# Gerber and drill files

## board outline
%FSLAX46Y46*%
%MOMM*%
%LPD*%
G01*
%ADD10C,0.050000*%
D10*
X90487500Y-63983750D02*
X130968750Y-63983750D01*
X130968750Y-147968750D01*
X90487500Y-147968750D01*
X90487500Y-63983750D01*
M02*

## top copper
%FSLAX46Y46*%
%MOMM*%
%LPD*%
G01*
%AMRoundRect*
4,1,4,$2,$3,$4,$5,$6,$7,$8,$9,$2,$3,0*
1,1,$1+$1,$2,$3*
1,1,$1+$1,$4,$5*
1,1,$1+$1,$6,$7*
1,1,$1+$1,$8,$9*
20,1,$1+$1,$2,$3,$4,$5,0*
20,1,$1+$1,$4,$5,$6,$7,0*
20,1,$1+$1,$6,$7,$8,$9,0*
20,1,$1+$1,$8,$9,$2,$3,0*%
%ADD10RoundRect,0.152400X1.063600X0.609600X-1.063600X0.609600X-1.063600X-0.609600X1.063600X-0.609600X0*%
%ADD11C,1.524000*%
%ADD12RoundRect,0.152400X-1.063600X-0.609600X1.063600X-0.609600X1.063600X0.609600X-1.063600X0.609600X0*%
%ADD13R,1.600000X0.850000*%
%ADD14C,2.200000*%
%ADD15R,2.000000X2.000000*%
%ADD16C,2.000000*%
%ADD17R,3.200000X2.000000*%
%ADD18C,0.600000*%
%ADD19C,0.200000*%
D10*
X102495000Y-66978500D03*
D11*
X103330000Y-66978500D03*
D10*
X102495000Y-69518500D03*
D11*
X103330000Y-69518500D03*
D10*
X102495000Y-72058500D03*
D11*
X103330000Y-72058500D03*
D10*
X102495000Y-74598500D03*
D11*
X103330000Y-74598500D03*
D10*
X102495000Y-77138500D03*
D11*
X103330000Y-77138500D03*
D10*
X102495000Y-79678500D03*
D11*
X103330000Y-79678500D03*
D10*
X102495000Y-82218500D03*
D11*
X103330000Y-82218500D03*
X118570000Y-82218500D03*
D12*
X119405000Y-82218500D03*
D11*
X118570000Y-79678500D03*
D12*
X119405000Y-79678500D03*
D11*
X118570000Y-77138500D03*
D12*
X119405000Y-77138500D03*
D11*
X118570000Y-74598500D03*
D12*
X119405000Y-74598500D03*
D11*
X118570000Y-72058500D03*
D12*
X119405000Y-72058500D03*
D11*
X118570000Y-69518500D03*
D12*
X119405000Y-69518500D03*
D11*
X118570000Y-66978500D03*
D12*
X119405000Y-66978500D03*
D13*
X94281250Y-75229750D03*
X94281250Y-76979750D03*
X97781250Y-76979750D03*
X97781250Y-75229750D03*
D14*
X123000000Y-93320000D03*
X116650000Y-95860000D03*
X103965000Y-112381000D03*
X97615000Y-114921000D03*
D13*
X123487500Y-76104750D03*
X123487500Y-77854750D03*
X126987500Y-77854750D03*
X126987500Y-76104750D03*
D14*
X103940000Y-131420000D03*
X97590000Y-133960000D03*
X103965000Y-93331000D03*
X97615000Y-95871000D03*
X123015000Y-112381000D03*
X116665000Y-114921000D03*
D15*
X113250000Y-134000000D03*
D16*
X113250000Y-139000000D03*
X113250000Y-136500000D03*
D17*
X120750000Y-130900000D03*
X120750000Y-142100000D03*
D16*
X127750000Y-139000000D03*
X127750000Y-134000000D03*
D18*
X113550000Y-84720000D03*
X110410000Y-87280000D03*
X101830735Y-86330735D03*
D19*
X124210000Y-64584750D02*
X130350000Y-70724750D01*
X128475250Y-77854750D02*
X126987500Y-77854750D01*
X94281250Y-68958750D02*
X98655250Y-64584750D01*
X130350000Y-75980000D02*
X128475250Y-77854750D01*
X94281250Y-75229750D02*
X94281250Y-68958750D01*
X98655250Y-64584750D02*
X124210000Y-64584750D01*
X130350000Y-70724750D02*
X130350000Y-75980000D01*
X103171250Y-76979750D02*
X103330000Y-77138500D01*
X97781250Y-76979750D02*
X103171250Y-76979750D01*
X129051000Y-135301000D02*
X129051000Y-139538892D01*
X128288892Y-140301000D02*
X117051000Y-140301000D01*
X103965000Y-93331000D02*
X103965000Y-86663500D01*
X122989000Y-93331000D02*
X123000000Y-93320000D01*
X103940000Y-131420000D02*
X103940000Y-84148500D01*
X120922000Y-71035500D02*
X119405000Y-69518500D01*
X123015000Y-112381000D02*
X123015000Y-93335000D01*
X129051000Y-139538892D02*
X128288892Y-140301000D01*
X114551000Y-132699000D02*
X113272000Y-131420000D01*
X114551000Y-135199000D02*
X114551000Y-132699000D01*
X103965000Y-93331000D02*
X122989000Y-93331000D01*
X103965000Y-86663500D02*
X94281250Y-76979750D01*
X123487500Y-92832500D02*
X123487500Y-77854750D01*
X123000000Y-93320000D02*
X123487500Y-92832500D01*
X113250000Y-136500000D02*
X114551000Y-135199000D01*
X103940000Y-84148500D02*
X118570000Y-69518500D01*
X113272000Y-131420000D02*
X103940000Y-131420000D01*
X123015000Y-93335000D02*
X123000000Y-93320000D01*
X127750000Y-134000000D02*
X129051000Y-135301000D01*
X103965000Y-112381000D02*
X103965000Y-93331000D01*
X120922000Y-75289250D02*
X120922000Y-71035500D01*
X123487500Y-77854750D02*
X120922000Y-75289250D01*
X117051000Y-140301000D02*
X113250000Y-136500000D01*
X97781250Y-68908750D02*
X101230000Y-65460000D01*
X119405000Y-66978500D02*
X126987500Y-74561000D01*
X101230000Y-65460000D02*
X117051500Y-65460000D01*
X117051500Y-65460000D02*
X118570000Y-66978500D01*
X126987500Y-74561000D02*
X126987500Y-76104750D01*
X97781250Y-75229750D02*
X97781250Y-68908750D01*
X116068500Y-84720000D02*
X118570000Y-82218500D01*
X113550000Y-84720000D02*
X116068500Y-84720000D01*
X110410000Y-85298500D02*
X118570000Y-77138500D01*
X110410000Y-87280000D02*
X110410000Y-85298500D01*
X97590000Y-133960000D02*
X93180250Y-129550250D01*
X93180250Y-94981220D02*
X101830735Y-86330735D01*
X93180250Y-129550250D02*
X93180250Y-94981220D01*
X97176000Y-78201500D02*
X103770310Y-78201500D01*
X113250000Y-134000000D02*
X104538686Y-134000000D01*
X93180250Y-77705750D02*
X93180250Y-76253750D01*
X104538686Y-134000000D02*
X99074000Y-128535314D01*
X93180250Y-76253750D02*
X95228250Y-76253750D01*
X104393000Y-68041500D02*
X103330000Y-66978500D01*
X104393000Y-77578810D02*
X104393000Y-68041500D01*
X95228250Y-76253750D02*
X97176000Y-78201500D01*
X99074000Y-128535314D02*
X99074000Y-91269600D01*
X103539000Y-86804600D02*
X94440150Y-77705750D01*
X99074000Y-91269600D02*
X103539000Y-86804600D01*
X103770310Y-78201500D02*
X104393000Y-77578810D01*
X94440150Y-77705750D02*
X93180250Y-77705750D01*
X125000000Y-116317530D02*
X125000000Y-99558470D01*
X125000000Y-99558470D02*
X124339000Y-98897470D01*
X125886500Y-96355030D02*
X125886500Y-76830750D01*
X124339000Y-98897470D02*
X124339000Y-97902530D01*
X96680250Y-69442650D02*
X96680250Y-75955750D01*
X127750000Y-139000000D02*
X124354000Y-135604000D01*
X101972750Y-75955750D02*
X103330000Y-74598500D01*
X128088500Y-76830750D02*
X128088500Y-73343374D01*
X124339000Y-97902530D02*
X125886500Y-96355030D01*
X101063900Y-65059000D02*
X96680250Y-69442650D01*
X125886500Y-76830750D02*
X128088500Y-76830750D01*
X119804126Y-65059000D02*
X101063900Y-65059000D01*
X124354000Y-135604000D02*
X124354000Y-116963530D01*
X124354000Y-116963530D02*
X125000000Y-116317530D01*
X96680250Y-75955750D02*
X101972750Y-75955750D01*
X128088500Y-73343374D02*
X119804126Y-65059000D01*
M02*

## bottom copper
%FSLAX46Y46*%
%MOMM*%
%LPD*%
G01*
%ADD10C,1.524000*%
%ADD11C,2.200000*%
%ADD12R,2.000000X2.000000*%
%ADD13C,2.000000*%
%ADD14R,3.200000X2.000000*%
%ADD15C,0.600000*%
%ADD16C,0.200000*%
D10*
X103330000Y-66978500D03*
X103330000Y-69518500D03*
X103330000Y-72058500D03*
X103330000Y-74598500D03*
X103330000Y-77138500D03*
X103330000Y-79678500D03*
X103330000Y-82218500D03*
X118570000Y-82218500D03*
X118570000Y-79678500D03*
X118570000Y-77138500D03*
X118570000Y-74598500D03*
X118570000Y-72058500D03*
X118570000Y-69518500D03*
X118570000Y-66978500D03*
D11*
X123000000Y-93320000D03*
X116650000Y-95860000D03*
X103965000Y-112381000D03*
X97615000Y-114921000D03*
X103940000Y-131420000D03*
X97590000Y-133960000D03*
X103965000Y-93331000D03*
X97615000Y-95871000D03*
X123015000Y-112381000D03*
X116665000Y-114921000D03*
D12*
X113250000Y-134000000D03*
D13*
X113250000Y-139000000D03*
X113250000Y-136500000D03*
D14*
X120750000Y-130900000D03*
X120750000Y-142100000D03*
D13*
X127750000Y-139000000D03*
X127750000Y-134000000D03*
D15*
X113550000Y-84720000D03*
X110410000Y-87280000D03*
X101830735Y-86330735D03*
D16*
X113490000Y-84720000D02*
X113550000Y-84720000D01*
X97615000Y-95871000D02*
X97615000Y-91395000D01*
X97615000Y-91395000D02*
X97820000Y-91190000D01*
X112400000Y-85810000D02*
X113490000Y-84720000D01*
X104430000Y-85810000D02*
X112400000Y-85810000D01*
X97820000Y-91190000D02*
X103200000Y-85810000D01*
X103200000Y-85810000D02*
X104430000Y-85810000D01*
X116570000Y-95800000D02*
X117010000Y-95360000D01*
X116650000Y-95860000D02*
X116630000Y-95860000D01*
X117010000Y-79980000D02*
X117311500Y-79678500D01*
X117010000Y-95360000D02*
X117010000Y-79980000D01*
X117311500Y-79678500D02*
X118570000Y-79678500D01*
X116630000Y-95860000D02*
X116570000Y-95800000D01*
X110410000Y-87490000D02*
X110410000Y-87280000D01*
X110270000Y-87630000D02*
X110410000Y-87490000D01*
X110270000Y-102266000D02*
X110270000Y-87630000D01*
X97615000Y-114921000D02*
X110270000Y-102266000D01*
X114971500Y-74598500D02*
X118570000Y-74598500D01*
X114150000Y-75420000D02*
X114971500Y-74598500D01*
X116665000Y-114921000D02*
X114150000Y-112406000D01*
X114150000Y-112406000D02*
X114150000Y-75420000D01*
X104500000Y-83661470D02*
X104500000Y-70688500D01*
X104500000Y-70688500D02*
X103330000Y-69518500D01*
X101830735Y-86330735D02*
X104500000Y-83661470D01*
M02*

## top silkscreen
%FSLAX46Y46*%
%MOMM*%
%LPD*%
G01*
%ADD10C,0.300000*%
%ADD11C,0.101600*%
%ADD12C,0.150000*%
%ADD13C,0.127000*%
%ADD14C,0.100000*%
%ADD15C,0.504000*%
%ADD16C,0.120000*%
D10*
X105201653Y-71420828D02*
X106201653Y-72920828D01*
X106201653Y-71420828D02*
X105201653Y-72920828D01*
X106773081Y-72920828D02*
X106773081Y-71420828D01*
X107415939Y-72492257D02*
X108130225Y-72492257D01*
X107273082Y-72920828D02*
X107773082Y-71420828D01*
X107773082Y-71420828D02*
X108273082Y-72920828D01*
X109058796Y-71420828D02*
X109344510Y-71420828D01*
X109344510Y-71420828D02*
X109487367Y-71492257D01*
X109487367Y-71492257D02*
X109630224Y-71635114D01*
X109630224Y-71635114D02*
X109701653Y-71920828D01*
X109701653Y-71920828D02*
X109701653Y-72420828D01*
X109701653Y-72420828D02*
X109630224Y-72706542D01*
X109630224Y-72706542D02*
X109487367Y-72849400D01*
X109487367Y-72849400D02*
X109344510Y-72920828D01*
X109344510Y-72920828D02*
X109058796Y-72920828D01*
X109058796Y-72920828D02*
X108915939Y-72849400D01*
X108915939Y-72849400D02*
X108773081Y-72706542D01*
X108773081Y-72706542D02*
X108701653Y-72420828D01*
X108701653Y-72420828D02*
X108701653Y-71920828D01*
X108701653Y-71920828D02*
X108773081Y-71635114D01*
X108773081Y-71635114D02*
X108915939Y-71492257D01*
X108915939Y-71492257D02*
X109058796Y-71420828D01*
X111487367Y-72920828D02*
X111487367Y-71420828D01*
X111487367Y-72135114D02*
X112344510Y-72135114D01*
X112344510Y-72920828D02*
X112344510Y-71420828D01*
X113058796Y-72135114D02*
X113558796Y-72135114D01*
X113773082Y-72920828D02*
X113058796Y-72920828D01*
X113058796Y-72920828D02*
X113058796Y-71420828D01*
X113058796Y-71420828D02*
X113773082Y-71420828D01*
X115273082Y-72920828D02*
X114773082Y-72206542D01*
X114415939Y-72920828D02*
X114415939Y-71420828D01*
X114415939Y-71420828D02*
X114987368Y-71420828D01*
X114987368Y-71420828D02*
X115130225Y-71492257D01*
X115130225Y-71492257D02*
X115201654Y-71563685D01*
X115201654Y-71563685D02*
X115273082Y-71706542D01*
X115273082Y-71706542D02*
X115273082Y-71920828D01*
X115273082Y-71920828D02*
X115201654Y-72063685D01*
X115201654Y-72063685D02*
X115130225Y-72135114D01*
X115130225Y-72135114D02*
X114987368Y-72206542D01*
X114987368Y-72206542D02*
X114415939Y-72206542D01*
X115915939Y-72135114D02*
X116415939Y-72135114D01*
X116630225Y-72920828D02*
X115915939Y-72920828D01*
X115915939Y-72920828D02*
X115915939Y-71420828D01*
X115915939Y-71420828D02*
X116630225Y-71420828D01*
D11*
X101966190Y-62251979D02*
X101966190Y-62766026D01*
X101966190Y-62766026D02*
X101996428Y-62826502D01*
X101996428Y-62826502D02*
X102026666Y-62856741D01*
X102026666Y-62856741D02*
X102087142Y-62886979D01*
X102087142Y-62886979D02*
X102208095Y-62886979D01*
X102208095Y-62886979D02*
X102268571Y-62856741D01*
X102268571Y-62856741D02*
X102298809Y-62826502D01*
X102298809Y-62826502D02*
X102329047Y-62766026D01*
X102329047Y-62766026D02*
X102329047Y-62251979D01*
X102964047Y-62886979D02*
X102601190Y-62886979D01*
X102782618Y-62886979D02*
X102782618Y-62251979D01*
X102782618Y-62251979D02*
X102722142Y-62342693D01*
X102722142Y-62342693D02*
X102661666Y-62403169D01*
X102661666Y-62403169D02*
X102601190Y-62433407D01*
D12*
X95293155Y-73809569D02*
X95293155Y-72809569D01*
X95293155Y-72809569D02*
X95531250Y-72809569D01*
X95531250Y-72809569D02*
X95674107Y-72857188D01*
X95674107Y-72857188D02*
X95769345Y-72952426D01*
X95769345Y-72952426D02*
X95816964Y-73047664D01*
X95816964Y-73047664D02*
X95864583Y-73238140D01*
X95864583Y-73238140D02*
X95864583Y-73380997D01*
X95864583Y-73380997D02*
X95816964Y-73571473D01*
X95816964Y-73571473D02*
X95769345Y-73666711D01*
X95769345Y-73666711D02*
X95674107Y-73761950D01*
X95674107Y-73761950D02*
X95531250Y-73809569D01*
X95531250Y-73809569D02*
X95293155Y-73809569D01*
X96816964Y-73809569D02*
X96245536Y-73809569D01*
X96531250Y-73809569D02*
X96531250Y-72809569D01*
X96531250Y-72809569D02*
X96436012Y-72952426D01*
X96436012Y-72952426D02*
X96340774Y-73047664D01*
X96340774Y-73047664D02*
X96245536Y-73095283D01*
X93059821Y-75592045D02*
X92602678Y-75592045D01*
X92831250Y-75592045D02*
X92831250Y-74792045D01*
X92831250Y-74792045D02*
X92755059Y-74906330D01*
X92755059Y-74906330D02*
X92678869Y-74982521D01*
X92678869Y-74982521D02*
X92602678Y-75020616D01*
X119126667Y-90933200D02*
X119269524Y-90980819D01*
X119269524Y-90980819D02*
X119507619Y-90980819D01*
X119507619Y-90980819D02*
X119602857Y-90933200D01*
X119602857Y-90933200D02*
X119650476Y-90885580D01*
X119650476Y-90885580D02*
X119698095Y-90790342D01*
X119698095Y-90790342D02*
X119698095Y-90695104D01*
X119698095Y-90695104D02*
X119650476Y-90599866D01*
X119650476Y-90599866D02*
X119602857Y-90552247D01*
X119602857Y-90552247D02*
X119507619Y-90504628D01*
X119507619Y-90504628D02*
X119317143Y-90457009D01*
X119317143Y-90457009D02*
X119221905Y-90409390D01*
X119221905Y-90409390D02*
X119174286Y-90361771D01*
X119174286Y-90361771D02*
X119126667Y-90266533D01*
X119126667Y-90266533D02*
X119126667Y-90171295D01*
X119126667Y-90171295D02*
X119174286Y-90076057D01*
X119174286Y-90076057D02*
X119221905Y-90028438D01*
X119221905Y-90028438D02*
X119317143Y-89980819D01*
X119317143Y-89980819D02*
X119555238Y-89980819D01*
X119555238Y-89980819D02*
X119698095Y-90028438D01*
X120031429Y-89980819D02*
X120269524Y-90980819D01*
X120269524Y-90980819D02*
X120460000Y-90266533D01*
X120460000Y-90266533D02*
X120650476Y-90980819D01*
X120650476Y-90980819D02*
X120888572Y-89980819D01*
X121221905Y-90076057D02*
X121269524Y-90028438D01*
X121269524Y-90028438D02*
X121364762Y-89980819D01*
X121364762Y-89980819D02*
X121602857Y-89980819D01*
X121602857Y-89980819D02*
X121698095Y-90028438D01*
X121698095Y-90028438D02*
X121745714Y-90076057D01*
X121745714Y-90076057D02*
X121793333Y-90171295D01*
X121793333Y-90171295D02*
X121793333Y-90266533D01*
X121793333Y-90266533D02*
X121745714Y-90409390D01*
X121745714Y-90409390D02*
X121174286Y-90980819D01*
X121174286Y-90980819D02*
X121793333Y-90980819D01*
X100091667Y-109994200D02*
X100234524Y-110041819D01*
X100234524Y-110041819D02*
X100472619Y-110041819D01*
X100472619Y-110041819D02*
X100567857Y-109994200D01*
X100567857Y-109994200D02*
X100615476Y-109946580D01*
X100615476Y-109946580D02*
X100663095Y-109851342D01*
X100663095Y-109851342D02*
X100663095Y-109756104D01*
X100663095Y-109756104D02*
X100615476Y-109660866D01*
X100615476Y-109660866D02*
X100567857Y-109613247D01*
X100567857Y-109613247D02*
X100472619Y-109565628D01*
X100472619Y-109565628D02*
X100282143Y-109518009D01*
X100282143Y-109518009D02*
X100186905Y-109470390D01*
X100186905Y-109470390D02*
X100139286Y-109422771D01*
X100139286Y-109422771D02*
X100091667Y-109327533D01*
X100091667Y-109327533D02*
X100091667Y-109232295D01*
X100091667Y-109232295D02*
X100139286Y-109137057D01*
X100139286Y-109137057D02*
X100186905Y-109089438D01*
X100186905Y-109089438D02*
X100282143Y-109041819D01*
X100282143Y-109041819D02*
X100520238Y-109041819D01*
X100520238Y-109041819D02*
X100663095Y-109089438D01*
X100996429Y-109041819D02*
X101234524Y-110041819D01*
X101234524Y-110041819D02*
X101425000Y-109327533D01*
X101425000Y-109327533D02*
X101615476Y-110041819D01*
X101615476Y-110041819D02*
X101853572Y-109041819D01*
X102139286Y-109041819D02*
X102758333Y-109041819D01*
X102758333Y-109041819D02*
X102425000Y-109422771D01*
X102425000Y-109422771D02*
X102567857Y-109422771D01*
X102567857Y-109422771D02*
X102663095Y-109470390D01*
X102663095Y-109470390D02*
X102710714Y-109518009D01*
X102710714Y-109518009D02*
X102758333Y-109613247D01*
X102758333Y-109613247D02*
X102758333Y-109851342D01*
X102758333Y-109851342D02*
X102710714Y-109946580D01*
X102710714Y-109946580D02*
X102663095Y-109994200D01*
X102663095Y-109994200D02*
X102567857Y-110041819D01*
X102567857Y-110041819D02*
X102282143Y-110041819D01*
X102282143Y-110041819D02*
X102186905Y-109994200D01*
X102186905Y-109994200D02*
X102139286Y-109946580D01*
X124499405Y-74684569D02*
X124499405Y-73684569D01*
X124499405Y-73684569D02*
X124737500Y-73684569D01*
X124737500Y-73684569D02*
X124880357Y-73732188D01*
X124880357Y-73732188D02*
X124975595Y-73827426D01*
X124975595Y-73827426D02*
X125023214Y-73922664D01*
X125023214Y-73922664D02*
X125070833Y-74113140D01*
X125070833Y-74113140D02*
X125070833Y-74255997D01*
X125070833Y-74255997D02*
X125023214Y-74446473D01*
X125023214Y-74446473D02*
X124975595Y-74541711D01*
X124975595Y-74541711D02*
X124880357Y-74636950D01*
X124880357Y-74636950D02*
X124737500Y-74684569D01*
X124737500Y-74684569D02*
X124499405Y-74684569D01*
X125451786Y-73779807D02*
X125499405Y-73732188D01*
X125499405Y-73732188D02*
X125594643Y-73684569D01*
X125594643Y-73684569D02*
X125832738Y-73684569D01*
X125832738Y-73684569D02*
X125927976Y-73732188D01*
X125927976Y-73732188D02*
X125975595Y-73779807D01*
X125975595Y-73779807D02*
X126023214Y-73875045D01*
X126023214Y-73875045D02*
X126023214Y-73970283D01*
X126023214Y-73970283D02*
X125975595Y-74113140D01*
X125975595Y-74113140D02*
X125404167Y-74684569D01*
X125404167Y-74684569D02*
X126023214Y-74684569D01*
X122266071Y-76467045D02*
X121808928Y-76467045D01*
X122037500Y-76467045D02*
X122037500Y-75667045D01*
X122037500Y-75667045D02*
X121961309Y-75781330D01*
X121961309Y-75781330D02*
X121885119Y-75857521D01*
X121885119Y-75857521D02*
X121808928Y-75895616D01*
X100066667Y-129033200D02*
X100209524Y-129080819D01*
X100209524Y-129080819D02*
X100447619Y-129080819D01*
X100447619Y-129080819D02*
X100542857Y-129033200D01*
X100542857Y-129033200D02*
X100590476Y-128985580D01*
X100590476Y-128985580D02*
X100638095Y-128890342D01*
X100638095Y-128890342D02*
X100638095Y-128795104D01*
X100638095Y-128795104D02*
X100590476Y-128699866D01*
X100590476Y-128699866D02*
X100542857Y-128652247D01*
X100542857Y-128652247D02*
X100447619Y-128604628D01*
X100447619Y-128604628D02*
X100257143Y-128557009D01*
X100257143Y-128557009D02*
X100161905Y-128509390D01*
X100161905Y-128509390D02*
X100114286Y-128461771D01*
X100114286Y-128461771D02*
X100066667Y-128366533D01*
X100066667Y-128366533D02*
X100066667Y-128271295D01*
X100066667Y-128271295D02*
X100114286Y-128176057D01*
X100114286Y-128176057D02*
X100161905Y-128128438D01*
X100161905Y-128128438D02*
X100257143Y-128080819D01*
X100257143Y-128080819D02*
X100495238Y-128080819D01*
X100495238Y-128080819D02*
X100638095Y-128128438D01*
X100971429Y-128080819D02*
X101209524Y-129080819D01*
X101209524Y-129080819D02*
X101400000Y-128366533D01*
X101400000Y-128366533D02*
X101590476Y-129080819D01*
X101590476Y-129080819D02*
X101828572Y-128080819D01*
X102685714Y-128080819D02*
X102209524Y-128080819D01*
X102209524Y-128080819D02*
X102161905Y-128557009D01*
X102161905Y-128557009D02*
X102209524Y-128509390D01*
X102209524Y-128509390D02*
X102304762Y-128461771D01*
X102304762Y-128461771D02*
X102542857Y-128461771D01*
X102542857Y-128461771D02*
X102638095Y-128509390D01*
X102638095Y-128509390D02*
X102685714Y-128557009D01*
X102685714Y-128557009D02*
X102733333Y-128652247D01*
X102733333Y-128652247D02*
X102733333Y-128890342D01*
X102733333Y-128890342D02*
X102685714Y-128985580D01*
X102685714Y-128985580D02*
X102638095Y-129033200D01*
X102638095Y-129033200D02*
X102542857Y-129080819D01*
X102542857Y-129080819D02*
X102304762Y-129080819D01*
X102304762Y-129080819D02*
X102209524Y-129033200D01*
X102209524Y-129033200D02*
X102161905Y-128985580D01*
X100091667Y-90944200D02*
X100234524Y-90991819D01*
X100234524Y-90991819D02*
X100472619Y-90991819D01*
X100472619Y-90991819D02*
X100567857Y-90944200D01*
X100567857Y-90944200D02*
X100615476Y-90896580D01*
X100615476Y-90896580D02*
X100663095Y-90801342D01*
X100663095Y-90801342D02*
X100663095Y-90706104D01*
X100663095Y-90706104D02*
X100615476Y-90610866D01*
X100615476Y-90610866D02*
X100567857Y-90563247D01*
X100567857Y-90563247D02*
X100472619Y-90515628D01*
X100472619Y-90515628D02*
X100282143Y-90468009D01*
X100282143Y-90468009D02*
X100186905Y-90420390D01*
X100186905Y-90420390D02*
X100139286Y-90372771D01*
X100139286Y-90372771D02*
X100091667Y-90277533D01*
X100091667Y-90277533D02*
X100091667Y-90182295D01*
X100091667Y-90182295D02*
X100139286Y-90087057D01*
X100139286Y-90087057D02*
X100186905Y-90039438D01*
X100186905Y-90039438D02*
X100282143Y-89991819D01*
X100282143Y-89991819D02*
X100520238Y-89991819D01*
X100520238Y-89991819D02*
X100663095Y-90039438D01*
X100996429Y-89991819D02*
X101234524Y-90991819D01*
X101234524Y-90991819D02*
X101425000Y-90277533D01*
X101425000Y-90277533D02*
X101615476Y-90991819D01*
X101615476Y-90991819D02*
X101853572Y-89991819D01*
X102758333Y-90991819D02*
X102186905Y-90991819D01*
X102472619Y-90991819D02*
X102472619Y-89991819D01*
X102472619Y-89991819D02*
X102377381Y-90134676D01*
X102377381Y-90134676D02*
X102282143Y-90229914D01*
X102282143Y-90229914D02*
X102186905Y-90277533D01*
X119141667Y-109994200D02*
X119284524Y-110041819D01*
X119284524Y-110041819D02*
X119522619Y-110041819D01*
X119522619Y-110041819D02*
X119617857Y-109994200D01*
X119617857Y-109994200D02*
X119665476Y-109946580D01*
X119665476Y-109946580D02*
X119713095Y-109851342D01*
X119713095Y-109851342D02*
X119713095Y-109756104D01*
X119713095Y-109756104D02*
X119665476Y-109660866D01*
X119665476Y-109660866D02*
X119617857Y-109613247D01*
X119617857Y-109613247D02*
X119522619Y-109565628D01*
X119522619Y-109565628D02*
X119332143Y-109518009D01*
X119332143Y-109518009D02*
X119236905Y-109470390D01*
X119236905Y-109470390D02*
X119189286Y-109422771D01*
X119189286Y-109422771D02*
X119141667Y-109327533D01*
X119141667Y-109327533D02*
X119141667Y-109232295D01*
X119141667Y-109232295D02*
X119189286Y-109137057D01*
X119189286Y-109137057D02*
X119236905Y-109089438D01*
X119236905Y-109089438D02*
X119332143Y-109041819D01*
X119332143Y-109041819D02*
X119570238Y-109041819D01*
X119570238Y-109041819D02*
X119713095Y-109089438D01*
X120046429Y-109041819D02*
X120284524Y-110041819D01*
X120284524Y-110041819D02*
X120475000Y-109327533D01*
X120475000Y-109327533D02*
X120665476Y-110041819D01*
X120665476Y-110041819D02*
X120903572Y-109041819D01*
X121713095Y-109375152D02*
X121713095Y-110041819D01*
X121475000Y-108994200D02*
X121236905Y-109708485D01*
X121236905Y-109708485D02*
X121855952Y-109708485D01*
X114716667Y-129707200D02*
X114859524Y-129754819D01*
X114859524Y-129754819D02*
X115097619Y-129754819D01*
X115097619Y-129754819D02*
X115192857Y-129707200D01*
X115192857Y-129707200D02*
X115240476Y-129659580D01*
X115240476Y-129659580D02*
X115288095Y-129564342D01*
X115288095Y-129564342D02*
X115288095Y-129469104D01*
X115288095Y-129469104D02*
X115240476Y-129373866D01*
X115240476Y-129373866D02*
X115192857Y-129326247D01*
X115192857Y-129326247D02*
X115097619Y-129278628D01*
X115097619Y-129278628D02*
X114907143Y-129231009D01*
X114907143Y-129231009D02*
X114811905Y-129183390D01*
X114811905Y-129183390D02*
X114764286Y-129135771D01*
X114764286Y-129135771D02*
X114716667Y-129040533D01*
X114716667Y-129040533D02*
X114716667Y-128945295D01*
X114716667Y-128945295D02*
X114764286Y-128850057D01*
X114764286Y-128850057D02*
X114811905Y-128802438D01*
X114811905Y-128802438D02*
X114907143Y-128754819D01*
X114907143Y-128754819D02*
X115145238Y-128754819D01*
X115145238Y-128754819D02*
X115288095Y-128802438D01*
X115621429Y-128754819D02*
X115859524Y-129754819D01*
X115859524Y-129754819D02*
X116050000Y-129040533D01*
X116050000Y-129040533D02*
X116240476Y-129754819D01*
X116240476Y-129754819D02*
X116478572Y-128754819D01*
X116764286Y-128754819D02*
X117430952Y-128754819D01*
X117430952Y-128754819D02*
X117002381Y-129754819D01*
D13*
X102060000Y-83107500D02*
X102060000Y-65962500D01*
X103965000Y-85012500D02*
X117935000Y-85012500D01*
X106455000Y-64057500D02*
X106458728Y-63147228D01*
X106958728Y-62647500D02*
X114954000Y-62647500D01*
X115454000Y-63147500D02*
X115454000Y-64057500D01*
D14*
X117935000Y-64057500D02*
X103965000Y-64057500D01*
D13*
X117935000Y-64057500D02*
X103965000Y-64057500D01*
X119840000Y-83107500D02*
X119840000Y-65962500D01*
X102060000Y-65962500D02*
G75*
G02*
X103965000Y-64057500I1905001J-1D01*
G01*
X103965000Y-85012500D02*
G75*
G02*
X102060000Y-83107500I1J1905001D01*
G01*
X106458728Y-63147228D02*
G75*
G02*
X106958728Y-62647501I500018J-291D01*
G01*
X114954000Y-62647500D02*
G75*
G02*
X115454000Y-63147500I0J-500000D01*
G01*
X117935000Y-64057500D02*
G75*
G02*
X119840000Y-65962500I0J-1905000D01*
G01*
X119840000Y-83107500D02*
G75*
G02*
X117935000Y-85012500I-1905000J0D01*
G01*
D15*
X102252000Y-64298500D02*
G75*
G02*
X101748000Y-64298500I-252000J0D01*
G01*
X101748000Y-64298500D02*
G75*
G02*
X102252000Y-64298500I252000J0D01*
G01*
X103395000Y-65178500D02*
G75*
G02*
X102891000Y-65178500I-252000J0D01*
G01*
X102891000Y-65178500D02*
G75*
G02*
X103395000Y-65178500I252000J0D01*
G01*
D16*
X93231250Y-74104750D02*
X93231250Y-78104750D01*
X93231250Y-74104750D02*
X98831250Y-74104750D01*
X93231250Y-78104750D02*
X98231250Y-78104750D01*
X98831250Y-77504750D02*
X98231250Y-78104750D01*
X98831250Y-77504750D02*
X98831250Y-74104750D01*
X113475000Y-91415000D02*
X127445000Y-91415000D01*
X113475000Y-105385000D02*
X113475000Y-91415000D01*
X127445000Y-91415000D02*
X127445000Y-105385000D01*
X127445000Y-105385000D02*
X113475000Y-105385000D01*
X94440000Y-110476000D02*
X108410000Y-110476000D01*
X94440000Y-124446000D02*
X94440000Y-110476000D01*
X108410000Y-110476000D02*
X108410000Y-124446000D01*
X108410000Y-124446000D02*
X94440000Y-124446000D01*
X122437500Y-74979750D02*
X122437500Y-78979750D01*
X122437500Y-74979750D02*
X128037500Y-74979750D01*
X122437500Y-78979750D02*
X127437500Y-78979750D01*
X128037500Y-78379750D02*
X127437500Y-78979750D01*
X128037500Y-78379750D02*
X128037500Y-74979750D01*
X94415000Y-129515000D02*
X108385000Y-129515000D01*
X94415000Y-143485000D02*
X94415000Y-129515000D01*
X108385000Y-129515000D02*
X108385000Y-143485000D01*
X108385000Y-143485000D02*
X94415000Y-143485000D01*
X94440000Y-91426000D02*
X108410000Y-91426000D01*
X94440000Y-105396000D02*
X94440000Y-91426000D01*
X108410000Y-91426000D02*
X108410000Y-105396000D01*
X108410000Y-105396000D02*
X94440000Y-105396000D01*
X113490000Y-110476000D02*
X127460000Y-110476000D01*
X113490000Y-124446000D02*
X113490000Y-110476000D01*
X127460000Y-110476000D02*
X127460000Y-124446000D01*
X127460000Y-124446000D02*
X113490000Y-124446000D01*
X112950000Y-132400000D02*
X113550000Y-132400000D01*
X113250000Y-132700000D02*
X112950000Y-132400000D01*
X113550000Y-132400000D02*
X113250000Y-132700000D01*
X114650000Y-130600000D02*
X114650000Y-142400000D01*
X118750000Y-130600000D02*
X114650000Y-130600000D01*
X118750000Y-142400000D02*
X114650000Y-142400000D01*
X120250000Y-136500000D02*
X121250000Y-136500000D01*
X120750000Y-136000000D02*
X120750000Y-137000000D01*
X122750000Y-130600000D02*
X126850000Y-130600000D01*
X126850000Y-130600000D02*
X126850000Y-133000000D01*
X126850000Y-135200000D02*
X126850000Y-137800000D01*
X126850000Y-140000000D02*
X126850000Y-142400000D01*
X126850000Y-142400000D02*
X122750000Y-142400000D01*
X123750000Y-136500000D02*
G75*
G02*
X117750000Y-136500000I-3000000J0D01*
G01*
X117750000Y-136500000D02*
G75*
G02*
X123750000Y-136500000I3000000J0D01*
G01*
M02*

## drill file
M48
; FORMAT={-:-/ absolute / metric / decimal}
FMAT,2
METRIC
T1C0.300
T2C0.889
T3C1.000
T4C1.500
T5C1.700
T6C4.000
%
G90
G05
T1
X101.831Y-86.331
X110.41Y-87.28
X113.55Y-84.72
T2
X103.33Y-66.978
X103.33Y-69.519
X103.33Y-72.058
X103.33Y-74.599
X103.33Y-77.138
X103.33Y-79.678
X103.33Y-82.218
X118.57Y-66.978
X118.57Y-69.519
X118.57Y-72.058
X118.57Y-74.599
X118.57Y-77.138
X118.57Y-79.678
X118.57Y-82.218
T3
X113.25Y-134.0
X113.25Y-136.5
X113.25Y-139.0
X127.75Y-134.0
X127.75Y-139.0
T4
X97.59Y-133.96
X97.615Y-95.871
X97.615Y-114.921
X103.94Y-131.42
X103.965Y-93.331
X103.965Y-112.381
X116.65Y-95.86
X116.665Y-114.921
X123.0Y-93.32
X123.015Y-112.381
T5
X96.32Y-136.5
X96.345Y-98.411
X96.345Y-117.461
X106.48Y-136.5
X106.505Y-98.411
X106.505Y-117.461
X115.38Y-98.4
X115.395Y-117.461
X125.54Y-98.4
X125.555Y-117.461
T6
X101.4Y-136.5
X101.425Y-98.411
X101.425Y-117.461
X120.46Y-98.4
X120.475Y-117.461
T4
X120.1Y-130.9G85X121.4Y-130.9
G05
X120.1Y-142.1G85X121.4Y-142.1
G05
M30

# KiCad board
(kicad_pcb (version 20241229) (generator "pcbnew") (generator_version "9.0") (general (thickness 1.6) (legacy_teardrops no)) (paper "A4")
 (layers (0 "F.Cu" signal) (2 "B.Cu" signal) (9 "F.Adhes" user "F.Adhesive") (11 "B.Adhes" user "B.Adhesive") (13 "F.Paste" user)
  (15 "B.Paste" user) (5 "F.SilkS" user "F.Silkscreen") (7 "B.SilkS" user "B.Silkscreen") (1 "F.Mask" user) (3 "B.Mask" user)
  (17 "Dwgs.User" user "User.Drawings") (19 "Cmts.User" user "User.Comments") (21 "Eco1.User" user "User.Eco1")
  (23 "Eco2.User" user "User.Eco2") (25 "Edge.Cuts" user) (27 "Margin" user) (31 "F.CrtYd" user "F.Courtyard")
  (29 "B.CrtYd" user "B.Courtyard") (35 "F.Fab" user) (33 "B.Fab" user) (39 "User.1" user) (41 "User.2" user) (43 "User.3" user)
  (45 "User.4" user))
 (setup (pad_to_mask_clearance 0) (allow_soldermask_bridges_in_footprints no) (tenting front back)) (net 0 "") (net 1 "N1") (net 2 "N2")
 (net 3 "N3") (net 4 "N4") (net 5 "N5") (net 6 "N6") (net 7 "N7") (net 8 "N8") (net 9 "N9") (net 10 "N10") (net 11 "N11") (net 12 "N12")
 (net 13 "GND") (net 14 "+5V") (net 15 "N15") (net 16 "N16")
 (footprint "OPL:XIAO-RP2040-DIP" (layer "F.Cu") (at 110.95 74.5985)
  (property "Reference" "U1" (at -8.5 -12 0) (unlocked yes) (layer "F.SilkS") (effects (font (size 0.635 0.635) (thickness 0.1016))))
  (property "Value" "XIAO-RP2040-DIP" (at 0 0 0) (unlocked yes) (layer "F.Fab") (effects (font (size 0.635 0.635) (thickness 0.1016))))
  (fp_line (start -8.89 8.509) (end -8.89 -8.636) (stroke (width 0.127) (type solid)) (layer "F.SilkS"))
  (fp_line (start -6.985 10.414) (end 6.985 10.414) (stroke (width 0.127) (type solid)) (layer "F.SilkS"))
  (fp_line (start -4.495 -10.541) (end -4.491272 -11.451272) (stroke (width 0.127) (type solid)) (layer "F.SilkS"))
  (fp_line (start -3.991272 -11.951) (end 4.004 -11.951) (stroke (width 0.127) (type solid)) (layer "F.SilkS"))
  (fp_line (start 4.504 -11.451) (end 4.504 -10.541) (stroke (width 0.127) (type solid)) (layer "F.SilkS"))
  (fp_line (start 6.985 -10.541) (end -6.985 -10.541) (stroke (width 0.1) (type solid)) (layer "F.SilkS"))
  (fp_line (start 6.985 -10.541) (end -6.985 -10.541) (stroke (width 0.127) (type solid)) (layer "F.SilkS"))
  (fp_line (start 8.89 8.509) (end 8.89 -8.636) (stroke (width 0.127) (type solid)) (layer "F.SilkS"))
  (fp_arc (start -8.89 -8.636) (mid -8.332038 -9.983038) (end -6.985 -10.541) (stroke (width 0.127) (type solid)) (layer "F.SilkS"))
  (fp_arc (start -6.985 10.414) (mid -8.332038 9.856038) (end -8.89 8.509) (stroke (width 0.127) (type solid)) (layer "F.SilkS"))
  (fp_arc (start -4.491272 -11.451272) (mid -4.344728 -11.80464) (end -3.991272 -11.951) (stroke (width 0.127) (type default))
   (layer "F.SilkS"))
  (fp_arc (start 4.004 -11.951) (mid 4.357553 -11.804553) (end 4.504 -11.451) (stroke (width 0.127) (type default)) (layer "F.SilkS"))
  (fp_arc (start 6.985 -10.541) (mid 8.332038 -9.983038) (end 8.89 -8.636) (stroke (width 0.127) (type solid)) (layer "F.SilkS"))
  (fp_arc (start 8.89 8.509) (mid 8.332038 9.856038) (end 6.985 10.414) (stroke (width 0.127) (type solid)) (layer "F.SilkS"))
  (fp_circle (center -8.95 -10.3) (end -8.95 -10.554) (stroke (width 0.5) (type solid)) (fill yes) (layer "F.SilkS"))
  (fp_circle (center -7.807 -9.42) (end -7.807 -9.674) (stroke (width 0.5) (type solid)) (fill yes) (layer "F.SilkS"))
  (pad "1" smd roundrect (at -8.455 -7.62 180) (size 2.432 1.524) (layers "F.Cu" "F.Mask") (roundrect_rratio 0.1) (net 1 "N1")
   (thermal_bridge_angle 45))
  (pad "1" thru_hole circle (at -7.62 -7.62 180) (size 1.524 1.524) (drill 0.889) (layers "*.Cu" "*.Mask") (remove_unused_layers no)
   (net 1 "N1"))
  (pad "2" smd roundrect (at -8.455 -5.08 180) (size 2.432 1.524) (layers "F.Cu" "F.Mask") (roundrect_rratio 0.1) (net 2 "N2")
   (thermal_bridge_angle 45))
  (pad "2" thru_hole circle (at -7.62 -5.08 180) (size 1.524 1.524) (drill 0.889) (layers "*.Cu" "*.Mask") (remove_unused_layers no)
   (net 2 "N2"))
  (pad "3" smd roundrect (at -8.455 -2.54 180) (size 2.432 1.524) (layers "F.Cu" "F.Mask") (roundrect_rratio 0.1) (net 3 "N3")
   (thermal_bridge_angle 45))
  (pad "3" thru_hole circle (at -7.62 -2.54 180) (size 1.524 1.524) (drill 0.889) (layers "*.Cu" "*.Mask") (remove_unused_layers no)
   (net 3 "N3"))
  (pad "4" smd roundrect (at -8.455 0 180) (size 2.432 1.524) (layers "F.Cu" "F.Mask") (roundrect_rratio 0.1) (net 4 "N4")
   (thermal_bridge_angle 45))
  (pad "4" thru_hole circle (at -7.62 0 180) (size 1.524 1.524) (drill 0.889) (layers "*.Cu" "*.Mask") (remove_unused_layers no)
   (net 4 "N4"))
  (pad "5" smd roundrect (at -8.455 2.54 180) (size 2.432 1.524) (layers "F.Cu" "F.Mask") (roundrect_rratio 0.1) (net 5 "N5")
   (thermal_bridge_angle 45))
  (pad "5" thru_hole circle (at -7.62 2.54 180) (size 1.524 1.524) (drill 0.889) (layers "*.Cu" "*.Mask") (remove_unused_layers no)
   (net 5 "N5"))
  (pad "6" smd roundrect (at -8.455 5.08 180) (size 2.432 1.524) (layers "F.Cu" "F.Mask") (roundrect_rratio 0.1) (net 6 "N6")
   (thermal_bridge_angle 45))
  (pad "6" thru_hole circle (at -7.62 5.08 180) (size 1.524 1.524) (drill 0.889) (layers "*.Cu" "*.Mask") (remove_unused_layers no)
   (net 6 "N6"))
  (pad "7" smd roundrect (at -8.455 7.62 180) (size 2.432 1.524) (layers "F.Cu" "F.Mask") (roundrect_rratio 0.1) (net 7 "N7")
   (thermal_bridge_angle 45))
  (pad "7" thru_hole circle (at -7.62 7.62 180) (size 1.524 1.524) (drill 0.889) (layers "*.Cu" "*.Mask") (remove_unused_layers no)
   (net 7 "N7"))
  (pad "8" thru_hole circle (at 7.62 7.62) (size 1.524 1.524) (drill 0.889) (layers "*.Cu" "*.Mask") (remove_unused_layers no) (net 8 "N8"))
  (pad "8" smd roundrect (at 8.455 7.62) (size 2.432 1.524) (layers "F.Cu" "F.Mask") (roundrect_rratio 0.1) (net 8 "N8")
   (thermal_bridge_angle 45))
  (pad "9" thru_hole circle (at 7.62 5.08) (size 1.524 1.524) (drill 0.889) (layers "*.Cu" "*.Mask") (remove_unused_layers no) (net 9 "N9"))
  (pad "9" smd roundrect (at 8.455 5.08) (size 2.432 1.524) (layers "F.Cu" "F.Mask") (roundrect_rratio 0.1) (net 9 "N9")
   (thermal_bridge_angle 45))
  (pad "10" thru_hole circle (at 7.62 2.54) (size 1.524 1.524) (drill 0.889) (layers "*.Cu" "*.Mask") (remove_unused_layers no)
   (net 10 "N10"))
  (pad "10" smd roundrect (at 8.455 2.54) (size 2.432 1.524) (layers "F.Cu" "F.Mask") (roundrect_rratio 0.1) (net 10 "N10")
   (thermal_bridge_angle 45))
  (pad "11" thru_hole circle (at 7.62 0) (size 1.524 1.524) (drill 0.889) (layers "*.Cu" "*.Mask") (remove_unused_layers no) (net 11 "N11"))
  (pad "11" smd roundrect (at 8.455 0) (size 2.432 1.524) (layers "F.Cu" "F.Mask") (roundrect_rratio 0.1) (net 11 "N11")
   (thermal_bridge_angle 45))
  (pad "12" thru_hole circle (at 7.62 -2.54) (size 1.524 1.524) (drill 0.889) (layers "*.Cu" "*.Mask") (remove_unused_layers no)
   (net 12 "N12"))
  (pad "12" smd roundrect (at 8.455 -2.54) (size 2.432 1.524) (layers "F.Cu" "F.Mask") (roundrect_rratio 0.1) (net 12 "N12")
   (thermal_bridge_angle 45))
  (pad "13" thru_hole circle (at 7.62 -5.08) (size 1.524 1.524) (drill 0.889) (layers "*.Cu" "*.Mask") (remove_unused_layers no)
   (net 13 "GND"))
  (pad "13" smd roundrect (at 8.455 -5.08) (size 2.432 1.524) (layers "F.Cu" "F.Mask") (roundrect_rratio 0.1) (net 13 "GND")
   (thermal_bridge_angle 45))
  (pad "14" thru_hole circle (at 7.62 -7.62) (size 1.524 1.524) (drill 0.889) (layers "*.Cu" "*.Mask") (remove_unused_layers no)
   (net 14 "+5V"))
  (pad "14" smd roundrect (at 8.455 -7.62) (size 2.432 1.524) (layers "F.Cu" "F.Mask") (roundrect_rratio 0.1) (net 14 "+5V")
   (thermal_bridge_angle 45)))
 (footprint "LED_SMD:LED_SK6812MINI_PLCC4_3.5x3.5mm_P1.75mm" (layer "F.Cu") (at 96.03125 76.10475)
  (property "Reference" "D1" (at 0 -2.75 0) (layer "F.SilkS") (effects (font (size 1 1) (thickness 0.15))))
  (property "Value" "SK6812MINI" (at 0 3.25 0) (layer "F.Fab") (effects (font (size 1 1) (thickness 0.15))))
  (fp_line (start -2.8 -2) (end -2.8 2) (stroke (width 0.12) (type default)) (layer "F.SilkS"))
  (fp_line (start -2.8 -2) (end 2.8 -2) (stroke (width 0.12) (type solid)) (layer "F.SilkS"))
  (fp_line (start -2.8 2) (end 2.2 2) (stroke (width 0.12) (type solid)) (layer "F.SilkS"))
  (fp_line (start 2.8 1.4) (end 2.2 2) (stroke (width 0.12) (type default)) (layer "F.SilkS"))
  (fp_line (start 2.8 1.4) (end 2.8 -2) (stroke (width 0.12) (type solid)) (layer "F.SilkS"))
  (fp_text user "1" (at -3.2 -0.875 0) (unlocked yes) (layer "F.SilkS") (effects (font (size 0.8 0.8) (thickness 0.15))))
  (pad "1" smd rect (at -1.75 -0.875) (size 1.6 0.85) (layers "F.Cu" "F.Mask" "F.Paste") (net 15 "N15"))
  (pad "2" smd rect (at -1.75 0.875) (size 1.6 0.85) (layers "F.Cu" "F.Mask" "F.Paste") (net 13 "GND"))
  (pad "3" smd rect (at 1.75 0.875) (size 1.6 0.85) (layers "F.Cu" "F.Mask" "F.Paste") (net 5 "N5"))
  (pad "4" smd rect (at 1.75 -0.875) (size 1.6 0.85) (layers "F.Cu" "F.Mask" "F.Paste") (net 14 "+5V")))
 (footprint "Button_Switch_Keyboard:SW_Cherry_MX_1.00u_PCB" (layer "F.Cu") (at 123 93.32)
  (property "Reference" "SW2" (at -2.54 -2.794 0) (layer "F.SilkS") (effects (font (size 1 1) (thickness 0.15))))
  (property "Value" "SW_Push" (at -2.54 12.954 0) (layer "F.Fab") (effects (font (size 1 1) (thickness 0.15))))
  (fp_line (start -9.525 -1.905) (end 4.445 -1.905) (stroke (width 0.12) (type solid)) (layer "F.SilkS"))
  (fp_line (start -9.525 12.065) (end -9.525 -1.905) (stroke (width 0.12) (type solid)) (layer "F.SilkS"))
  (fp_line (start 4.445 -1.905) (end 4.445 12.065) (stroke (width 0.12) (type solid)) (layer "F.SilkS"))
  (fp_line (start 4.445 12.065) (end -9.525 12.065) (stroke (width 0.12) (type solid)) (layer "F.SilkS"))
  (pad "" np_thru_hole circle (at -7.62 5.08) (size 1.7 1.7) (drill 1.7) (layers "*.Cu" "*.Mask"))
  (pad "" np_thru_hole circle (at -2.54 5.08) (size 4 4) (drill 4) (layers "*.Cu" "*.Mask"))
  (pad "" np_thru_hole circle (at 2.54 5.08) (size 1.7 1.7) (drill 1.7) (layers "*.Cu" "*.Mask"))
  (pad "1" thru_hole circle (at 0 0) (size 2.2 2.2) (drill 1.5) (layers "*.Cu" "*.Mask") (remove_unused_layers no) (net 13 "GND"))
  (pad "2" thru_hole circle (at -6.35 2.54) (size 2.2 2.2) (drill 1.5) (layers "*.Cu" "*.Mask") (remove_unused_layers no) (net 9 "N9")))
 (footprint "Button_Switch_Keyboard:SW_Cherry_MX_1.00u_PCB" (layer "F.Cu") (at 103.965 112.381)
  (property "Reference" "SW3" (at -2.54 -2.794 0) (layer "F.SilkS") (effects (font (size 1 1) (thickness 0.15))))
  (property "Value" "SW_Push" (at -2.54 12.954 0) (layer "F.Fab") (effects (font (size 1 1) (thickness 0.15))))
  (fp_line (start -9.525 -1.905) (end 4.445 -1.905) (stroke (width 0.12) (type solid)) (layer "F.SilkS"))
  (fp_line (start -9.525 12.065) (end -9.525 -1.905) (stroke (width 0.12) (type solid)) (layer "F.SilkS"))
  (fp_line (start 4.445 -1.905) (end 4.445 12.065) (stroke (width 0.12) (type solid)) (layer "F.SilkS"))
  (fp_line (start 4.445 12.065) (end -9.525 12.065) (stroke (width 0.12) (type solid)) (layer "F.SilkS"))
  (pad "" np_thru_hole circle (at -7.62 5.08) (size 1.7 1.7) (drill 1.7) (layers "*.Cu" "*.Mask"))
  (pad "" np_thru_hole circle (at -2.54 5.08) (size 4 4) (drill 4) (layers "*.Cu" "*.Mask"))
  (pad "" np_thru_hole circle (at 2.54 5.08) (size 1.7 1.7) (drill 1.7) (layers "*.Cu" "*.Mask"))
  (pad "1" thru_hole circle (at 0 0) (size 2.2 2.2) (drill 1.5) (layers "*.Cu" "*.Mask") (remove_unused_layers no) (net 13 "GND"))
  (pad "2" thru_hole circle (at -6.35 2.54) (size 2.2 2.2) (drill 1.5) (layers "*.Cu" "*.Mask") (remove_unused_layers no) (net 10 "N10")))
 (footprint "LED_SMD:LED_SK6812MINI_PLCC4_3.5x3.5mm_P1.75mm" (layer "F.Cu") (at 125.2375 76.97975)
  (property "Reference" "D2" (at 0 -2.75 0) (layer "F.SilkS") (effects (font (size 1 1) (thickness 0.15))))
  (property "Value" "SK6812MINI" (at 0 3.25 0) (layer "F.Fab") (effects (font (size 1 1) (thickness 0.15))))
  (fp_line (start -2.8 -2) (end -2.8 2) (stroke (width 0.12) (type default)) (layer "F.SilkS"))
  (fp_line (start -2.8 -2) (end 2.8 -2) (stroke (width 0.12) (type solid)) (layer "F.SilkS"))
  (fp_line (start -2.8 2) (end 2.2 2) (stroke (width 0.12) (type solid)) (layer "F.SilkS"))
  (fp_line (start 2.8 1.4) (end 2.2 2) (stroke (width 0.12) (type default)) (layer "F.SilkS"))
  (fp_line (start 2.8 1.4) (end 2.8 -2) (stroke (width 0.12) (type solid)) (layer "F.SilkS"))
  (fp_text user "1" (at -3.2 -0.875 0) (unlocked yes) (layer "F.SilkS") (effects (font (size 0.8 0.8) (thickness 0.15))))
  (pad "1" smd rect (at -1.75 -0.875) (size 1.6 0.85) (layers "F.Cu" "F.Mask" "F.Paste") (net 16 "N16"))
  (pad "2" smd rect (at -1.75 0.875) (size 1.6 0.85) (layers "F.Cu" "F.Mask" "F.Paste") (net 13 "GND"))
  (pad "3" smd rect (at 1.75 0.875) (size 1.6 0.85) (layers "F.Cu" "F.Mask" "F.Paste") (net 15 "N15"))
  (pad "4" smd rect (at 1.75 -0.875) (size 1.6 0.85) (layers "F.Cu" "F.Mask" "F.Paste") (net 14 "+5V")))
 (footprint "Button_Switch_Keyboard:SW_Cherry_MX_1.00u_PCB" (layer "F.Cu") (at 103.94 131.42)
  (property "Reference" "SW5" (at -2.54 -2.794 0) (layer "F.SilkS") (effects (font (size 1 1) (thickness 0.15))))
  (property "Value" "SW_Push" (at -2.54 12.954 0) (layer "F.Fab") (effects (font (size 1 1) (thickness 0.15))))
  (fp_line (start -9.525 -1.905) (end 4.445 -1.905) (stroke (width 0.12) (type solid)) (layer "F.SilkS"))
  (fp_line (start -9.525 12.065) (end -9.525 -1.905) (stroke (width 0.12) (type solid)) (layer "F.SilkS"))
  (fp_line (start 4.445 -1.905) (end 4.445 12.065) (stroke (width 0.12) (type solid)) (layer "F.SilkS"))
  (fp_line (start 4.445 12.065) (end -9.525 12.065) (stroke (width 0.12) (type solid)) (layer "F.SilkS"))
  (pad "" np_thru_hole circle (at -7.62 5.08) (size 1.7 1.7) (drill 1.7) (layers "*.Cu" "*.Mask"))
  (pad "" np_thru_hole circle (at -2.54 5.08) (size 4 4) (drill 4) (layers "*.Cu" "*.Mask"))
  (pad "" np_thru_hole circle (at 2.54 5.08) (size 1.7 1.7) (drill 1.7) (layers "*.Cu" "*.Mask"))
  (pad "1" thru_hole circle (at 0 0) (size 2.2 2.2) (drill 1.5) (layers "*.Cu" "*.Mask") (remove_unused_layers no) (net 13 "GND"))
  (pad "2" thru_hole circle (at -6.35 2.54) (size 2.2 2.2) (drill 1.5) (layers "*.Cu" "*.Mask") (remove_unused_layers no) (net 2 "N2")))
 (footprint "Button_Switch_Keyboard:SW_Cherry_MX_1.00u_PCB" (layer "F.Cu") (at 103.965 93.331)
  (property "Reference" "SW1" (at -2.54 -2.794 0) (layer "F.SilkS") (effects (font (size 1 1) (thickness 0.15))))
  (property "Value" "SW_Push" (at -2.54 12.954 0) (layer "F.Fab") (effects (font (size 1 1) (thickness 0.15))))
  (fp_line (start -9.525 -1.905) (end 4.445 -1.905) (stroke (width 0.12) (type solid)) (layer "F.SilkS"))
  (fp_line (start -9.525 12.065) (end -9.525 -1.905) (stroke (width 0.12) (type solid)) (layer "F.SilkS"))
  (fp_line (start 4.445 -1.905) (end 4.445 12.065) (stroke (width 0.12) (type solid)) (layer "F.SilkS"))
  (fp_line (start 4.445 12.065) (end -9.525 12.065) (stroke (width 0.12) (type solid)) (layer "F.SilkS"))
  (pad "" np_thru_hole circle (at -7.62 5.08) (size 1.7 1.7) (drill 1.7) (layers "*.Cu" "*.Mask"))
  (pad "" np_thru_hole circle (at -2.54 5.08) (size 4 4) (drill 4) (layers "*.Cu" "*.Mask"))
  (pad "" np_thru_hole circle (at 2.54 5.08) (size 1.7 1.7) (drill 1.7) (layers "*.Cu" "*.Mask"))
  (pad "1" thru_hole circle (at 0 0) (size 2.2 2.2) (drill 1.5) (layers "*.Cu" "*.Mask") (remove_unused_layers no) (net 13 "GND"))
  (pad "2" thru_hole circle (at -6.35 2.54) (size 2.2 2.2) (drill 1.5) (layers "*.Cu" "*.Mask") (remove_unused_layers no) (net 8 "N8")))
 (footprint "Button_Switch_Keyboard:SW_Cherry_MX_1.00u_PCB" (layer "F.Cu") (at 123.015 112.381)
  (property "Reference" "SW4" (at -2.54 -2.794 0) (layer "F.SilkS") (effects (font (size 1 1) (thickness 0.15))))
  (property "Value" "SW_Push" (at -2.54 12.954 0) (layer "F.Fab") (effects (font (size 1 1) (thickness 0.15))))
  (fp_line (start -9.525 -1.905) (end 4.445 -1.905) (stroke (width 0.12) (type solid)) (layer "F.SilkS"))
  (fp_line (start -9.525 12.065) (end -9.525 -1.905) (stroke (width 0.12) (type solid)) (layer "F.SilkS"))
  (fp_line (start 4.445 -1.905) (end 4.445 12.065) (stroke (width 0.12) (type solid)) (layer "F.SilkS"))
  (fp_line (start 4.445 12.065) (end -9.525 12.065) (stroke (width 0.12) (type solid)) (layer "F.SilkS"))
  (pad "" np_thru_hole circle (at -7.62 5.08) (size 1.7 1.7) (drill 1.7) (layers "*.Cu" "*.Mask"))
  (pad "" np_thru_hole circle (at -2.54 5.08) (size 4 4) (drill 4) (layers "*.Cu" "*.Mask"))
  (pad "" np_thru_hole circle (at 2.54 5.08) (size 1.7 1.7) (drill 1.7) (layers "*.Cu" "*.Mask"))
  (pad "1" thru_hole circle (at 0 0) (size 2.2 2.2) (drill 1.5) (layers "*.Cu" "*.Mask") (remove_unused_layers no) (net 13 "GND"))
  (pad "2" thru_hole circle (at -6.35 2.54) (size 2.2 2.2) (drill 1.5) (layers "*.Cu" "*.Mask") (remove_unused_layers no) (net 11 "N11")))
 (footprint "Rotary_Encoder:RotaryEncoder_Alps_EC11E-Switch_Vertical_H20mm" (layer "F.Cu") (at 113.25 134)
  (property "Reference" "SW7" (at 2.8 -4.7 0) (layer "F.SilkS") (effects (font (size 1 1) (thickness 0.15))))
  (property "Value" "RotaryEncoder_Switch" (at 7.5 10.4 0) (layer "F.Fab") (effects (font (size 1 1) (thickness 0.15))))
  (fp_line (start -0.3 -1.6) (end 0.3 -1.6) (stroke (width 0.12) (type solid)) (layer "F.SilkS"))
  (fp_line (start 0 -1.3) (end -0.3 -1.6) (stroke (width 0.12) (type solid)) (layer "F.SilkS"))
  (fp_line (start 0.3 -1.6) (end 0 -1.3) (stroke (width 0.12) (type solid)) (layer "F.SilkS"))
  (fp_line (start 1.4 -3.4) (end 1.4 8.4) (stroke (width 0.12) (type solid)) (layer "F.SilkS"))
  (fp_line (start 5.5 -3.4) (end 1.4 -3.4) (stroke (width 0.12) (type solid)) (layer "F.SilkS"))
  (fp_line (start 5.5 8.4) (end 1.4 8.4) (stroke (width 0.12) (type solid)) (layer "F.SilkS"))
  (fp_line (start 7 2.5) (end 8 2.5) (stroke (width 0.12) (type solid)) (layer "F.SilkS"))
  (fp_line (start 7.5 2) (end 7.5 3) (stroke (width 0.12) (type solid)) (layer "F.SilkS"))
  (fp_line (start 9.5 -3.4) (end 13.6 -3.4) (stroke (width 0.12) (type solid)) (layer "F.SilkS"))
  (fp_line (start 13.6 -3.4) (end 13.6 -1) (stroke (width 0.12) (type solid)) (layer "F.SilkS"))
  (fp_line (start 13.6 1.2) (end 13.6 3.8) (stroke (width 0.12) (type solid)) (layer "F.SilkS"))
  (fp_line (start 13.6 6) (end 13.6 8.4) (stroke (width 0.12) (type solid)) (layer "F.SilkS"))
  (fp_line (start 13.6 8.4) (end 9.5 8.4) (stroke (width 0.12) (type solid)) (layer "F.SilkS"))
  (fp_circle (center 7.5 2.5) (end 10.5 2.5) (stroke (width 0.12) (type solid)) (fill no) (layer "F.SilkS"))
  (pad "A" thru_hole rect (at 0 0) (size 2 2) (drill 1) (layers "*.Cu" "*.Mask") (remove_unused_layers no) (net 1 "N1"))
  (pad "B" thru_hole circle (at 0 5) (size 2 2) (drill 1) (layers "*.Cu" "*.Mask") (remove_unused_layers no) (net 3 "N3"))
  (pad "C" thru_hole circle (at 0 2.5) (size 2 2) (drill 1) (layers "*.Cu" "*.Mask") (remove_unused_layers no) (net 13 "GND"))
  (pad "MP" thru_hole rect (at 7.5 -3.1) (size 3.2 2) (drill oval 2.8 1.5) (layers "*.Cu" "*.Mask") (remove_unused_layers no))
  (pad "MP" thru_hole rect (at 7.5 8.1) (size 3.2 2) (drill oval 2.8 1.5) (layers "*.Cu" "*.Mask") (remove_unused_layers no))
  (pad "S1" thru_hole circle (at 14.5 5) (size 2 2) (drill 1) (layers "*.Cu" "*.Mask") (remove_unused_layers no) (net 4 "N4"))
  (pad "S2" thru_hole circle (at 14.5 0) (size 2 2) (drill 1) (layers "*.Cu" "*.Mask") (remove_unused_layers no) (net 13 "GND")))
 (gr_rect (start 90.4875 63.98375) (end 130.96875 147.96875) (stroke (width 0.05) (type default)) (fill no) (layer "Edge.Cuts"))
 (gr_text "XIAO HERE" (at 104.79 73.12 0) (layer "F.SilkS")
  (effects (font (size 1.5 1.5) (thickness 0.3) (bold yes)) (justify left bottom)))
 (segment (start 124.21 64.58475) (end 130.35 70.72475) (width 0.2) (layer "F.Cu") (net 15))
 (segment (start 128.47525 77.85475) (end 126.9875 77.85475) (width 0.2) (layer "F.Cu") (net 15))
 (segment (start 94.28125 68.95875) (end 98.65525 64.58475) (width 0.2) (layer "F.Cu") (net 15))
 (segment (start 130.35 75.98) (end 128.47525 77.85475) (width 0.2) (layer "F.Cu") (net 15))
 (segment (start 94.28125 75.22975) (end 94.28125 68.95875) (width 0.2) (layer "F.Cu") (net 15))
 (segment (start 98.65525 64.58475) (end 124.21 64.58475) (width 0.2) (layer "F.Cu") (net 15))
 (segment (start 130.35 70.72475) (end 130.35 75.98) (width 0.2) (layer "F.Cu") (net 15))
 (segment (start 103.17125 76.97975) (end 103.33 77.1385) (width 0.2) (layer "F.Cu") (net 5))
 (segment (start 97.78125 76.97975) (end 103.17125 76.97975) (width 0.2) (layer "F.Cu") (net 5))
 (segment (start 129.051 135.301) (end 129.051 139.538892) (width 0.2) (layer "F.Cu") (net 13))
 (segment (start 128.288892 140.301) (end 117.051 140.301) (width 0.2) (layer "F.Cu") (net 13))
 (segment (start 103.965 93.331) (end 103.965 86.6635) (width 0.2) (layer "F.Cu") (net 13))
 (segment (start 122.989 93.331) (end 123 93.32) (width 0.2) (layer "F.Cu") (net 13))
 (segment (start 103.94 131.42) (end 103.94 84.1485) (width 0.2) (layer "F.Cu") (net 13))
 (segment (start 120.922 71.0355) (end 119.405 69.5185) (width 0.2) (layer "F.Cu") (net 13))
 (segment (start 123.015 112.381) (end 123.015 93.335) (width 0.2) (layer "F.Cu") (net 13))
 (segment (start 129.051 139.538892) (end 128.288892 140.301) (width 0.2) (layer "F.Cu") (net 13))
 (segment (start 114.551 132.699) (end 113.272 131.42) (width 0.2) (layer "F.Cu") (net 13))
 (segment (start 114.551 135.199) (end 114.551 132.699) (width 0.2) (layer "F.Cu") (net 13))
 (segment (start 103.965 93.331) (end 122.989 93.331) (width 0.2) (layer "F.Cu") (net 13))
 (segment (start 103.965 86.6635) (end 94.28125 76.97975) (width 0.2) (layer "F.Cu") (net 13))
 (segment (start 123.4875 92.8325) (end 123.4875 77.85475) (width 0.2) (layer "F.Cu") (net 13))
 (segment (start 123 93.32) (end 123.4875 92.8325) (width 0.2) (layer "F.Cu") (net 13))
 (segment (start 113.25 136.5) (end 114.551 135.199) (width 0.2) (layer "F.Cu") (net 13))
 (segment (start 103.94 84.1485) (end 118.57 69.5185) (width 0.2) (layer "F.Cu") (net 13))
 (segment (start 113.272 131.42) (end 103.94 131.42) (width 0.2) (layer "F.Cu") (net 13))
 (segment (start 123.015 93.335) (end 123 93.32) (width 0.2) (layer "F.Cu") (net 13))
 (segment (start 127.75 134) (end 129.051 135.301) (width 0.2) (layer "F.Cu") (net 13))
 (segment (start 103.965 112.381) (end 103.965 93.331) (width 0.2) (layer "F.Cu") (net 13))
 (segment (start 120.922 75.28925) (end 120.922 71.0355) (width 0.2) (layer "F.Cu") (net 13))
 (segment (start 123.4875 77.85475) (end 120.922 75.28925) (width 0.2) (layer "F.Cu") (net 13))
 (segment (start 117.051 140.301) (end 113.25 136.5) (width 0.2) (layer "F.Cu") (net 13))
 (segment (start 97.78125 68.90875) (end 101.23 65.46) (width 0.2) (layer "F.Cu") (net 14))
 (segment (start 119.405 66.9785) (end 126.9875 74.561) (width 0.2) (layer "F.Cu") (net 14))
 (segment (start 101.23 65.46) (end 117.0515 65.46) (width 0.2) (layer "F.Cu") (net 14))
 (segment (start 117.0515 65.46) (end 118.57 66.9785) (width 0.2) (layer "F.Cu") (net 14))
 (segment (start 126.9875 74.561) (end 126.9875 76.10475) (width 0.2) (layer "F.Cu") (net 14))
 (segment (start 97.78125 75.22975) (end 97.78125 68.90875) (width 0.2) (layer "F.Cu") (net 14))
 (segment (start 116.0685 84.72) (end 118.57 82.2185) (width 0.2) (layer "F.Cu") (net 8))
 (segment (start 113.55 84.72) (end 116.0685 84.72) (width 0.2) (layer "F.Cu") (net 8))
 (via (at 113.55 84.72) (size 0.6) (drill 0.3) (layers "F.Cu" "B.Cu") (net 8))
 (segment (start 113.49 84.72) (end 113.55 84.72) (width 0.2) (layer "B.Cu") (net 8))
 (segment (start 97.615 95.871) (end 97.615 91.395) (width 0.2) (layer "B.Cu") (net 8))
 (segment (start 97.615 91.395) (end 97.82 91.19) (width 0.2) (layer "B.Cu") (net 8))
 (segment (start 112.4 85.81) (end 113.49 84.72) (width 0.2) (layer "B.Cu") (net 8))
 (segment (start 104.43 85.81) (end 112.4 85.81) (width 0.2) (layer "B.Cu") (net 8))
 (segment (start 97.82 91.19) (end 103.2 85.81) (width 0.2) (layer "B.Cu") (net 8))
 (segment (start 103.2 85.81) (end 104.43 85.81) (width 0.2) (layer "B.Cu") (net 8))
 (segment (start 116.57 95.8) (end 117.01 95.36) (width 0.2) (layer "B.Cu") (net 9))
 (segment (start 116.65 95.86) (end 116.63 95.86) (width 0.2) (layer "B.Cu") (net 9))
 (segment (start 117.01 79.98) (end 117.3115 79.6785) (width 0.2) (layer "B.Cu") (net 9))
 (segment (start 117.01 95.36) (end 117.01 79.98) (width 0.2) (layer "B.Cu") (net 9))
 (segment (start 117.3115 79.6785) (end 118.57 79.6785) (width 0.2) (layer "B.Cu") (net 9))
 (segment (start 116.63 95.86) (end 116.57 95.8) (width 0.2) (layer "B.Cu") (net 9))
 (segment (start 110.41 85.2985) (end 118.57 77.1385) (width 0.2) (layer "F.Cu") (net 10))
 (segment (start 110.41 87.28) (end 110.41 85.2985) (width 0.2) (layer "F.Cu") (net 10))
 (via (at 110.41 87.28) (size 0.6) (drill 0.3) (layers "F.Cu" "B.Cu") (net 10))
 (segment (start 110.41 87.49) (end 110.41 87.28) (width 0.2) (layer "B.Cu") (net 10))
 (segment (start 110.27 87.63) (end 110.41 87.49) (width 0.2) (layer "B.Cu") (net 10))
 (segment (start 110.27 102.266) (end 110.27 87.63) (width 0.2) (layer "B.Cu") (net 10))
 (segment (start 97.615 114.921) (end 110.27 102.266) (width 0.2) (layer "B.Cu") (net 10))
 (segment (start 114.9715 74.5985) (end 118.57 74.5985) (width 0.2) (layer "B.Cu") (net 11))
 (segment (start 114.15 75.42) (end 114.9715 74.5985) (width 0.2) (layer "B.Cu") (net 11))
 (segment (start 116.665 114.921) (end 114.15 112.406) (width 0.2) (layer "B.Cu") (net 11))
 (segment (start 114.15 112.406) (end 114.15 75.42) (width 0.2) (layer "B.Cu") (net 11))
 (segment (start 97.59 133.96) (end 93.18025 129.55025) (width 0.2) (layer "F.Cu") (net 2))
 (segment (start 93.18025 94.98122) (end 101.830735 86.330735) (width 0.2) (layer "F.Cu") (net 2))
 (segment (start 93.18025 129.55025) (end 93.18025 94.98122) (width 0.2) (layer "F.Cu") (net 2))
 (via (at 101.830735 86.330735) (size 0.6) (drill 0.3) (layers "F.Cu" "B.Cu") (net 2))
 (segment (start 104.5 83.66147) (end 104.5 70.6885) (width 0.2) (layer "B.Cu") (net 2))
 (segment (start 104.5 70.6885) (end 103.33 69.5185) (width 0.2) (layer "B.Cu") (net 2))
 (segment (start 101.830735 86.330735) (end 104.5 83.66147) (width 0.2) (layer "B.Cu") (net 2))
 (segment (start 97.176 78.2015) (end 103.77031 78.2015) (width 0.2) (layer "F.Cu") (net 1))
 (segment (start 113.25 134) (end 104.538686 134) (width 0.2) (layer "F.Cu") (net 1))
 (segment (start 93.18025 77.70575) (end 93.18025 76.25375) (width 0.2) (layer "F.Cu") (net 1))
 (segment (start 104.538686 134) (end 99.074 128.535314) (width 0.2) (layer "F.Cu") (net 1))
 (segment (start 93.18025 76.25375) (end 95.22825 76.25375) (width 0.2) (layer "F.Cu") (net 1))
 (segment (start 104.393 68.0415) (end 103.33 66.9785) (width 0.2) (layer "F.Cu") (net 1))
 (segment (start 104.393 77.57881) (end 104.393 68.0415) (width 0.2) (layer "F.Cu") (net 1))
 (segment (start 95.22825 76.25375) (end 97.176 78.2015) (width 0.2) (layer "F.Cu") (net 1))
 (segment (start 99.074 128.535314) (end 99.074 91.2696) (width 0.2) (layer "F.Cu") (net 1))
 (segment (start 103.539 86.8046) (end 94.44015 77.70575) (width 0.2) (layer "F.Cu") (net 1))
 (segment (start 99.074 91.2696) (end 103.539 86.8046) (width 0.2) (layer "F.Cu") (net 1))
 (segment (start 103.77031 78.2015) (end 104.393 77.57881) (width 0.2) (layer "F.Cu") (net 1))
 (segment (start 94.44015 77.70575) (end 93.18025 77.70575) (width 0.2) (layer "F.Cu") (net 1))
 (segment (start 125 116.31753) (end 125 99.55847) (width 0.2) (layer "F.Cu") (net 4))
 (segment (start 125 99.55847) (end 124.339 98.89747) (width 0.2) (layer "F.Cu") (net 4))
 (segment (start 125.8865 96.35503) (end 125.8865 76.83075) (width 0.2) (layer "F.Cu") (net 4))
 (segment (start 124.339 98.89747) (end 124.339 97.90253) (width 0.2) (layer "F.Cu") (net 4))
 (segment (start 96.68025 69.44265) (end 96.68025 75.95575) (width 0.2) (layer "F.Cu") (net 4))
 (segment (start 127.75 139) (end 124.354 135.604) (width 0.2) (layer "F.Cu") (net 4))
 (segment (start 101.97275 75.95575) (end 103.33 74.5985) (width 0.2) (layer "F.Cu") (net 4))
 (segment (start 128.0885 76.83075) (end 128.0885 73.343374) (width 0.2) (layer "F.Cu") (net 4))
 (segment (start 124.339 97.90253) (end 125.8865 96.35503) (width 0.2) (layer "F.Cu") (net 4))
 (segment (start 101.0639 65.059) (end 96.68025 69.44265) (width 0.2) (layer "F.Cu") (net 4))
 (segment (start 125.8865 76.83075) (end 128.0885 76.83075) (width 0.2) (layer "F.Cu") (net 4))
 (segment (start 119.804126 65.059) (end 101.0639 65.059) (width 0.2) (layer "F.Cu") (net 4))
 (segment (start 124.354 135.604) (end 124.354 116.96353) (width 0.2) (layer "F.Cu") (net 4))
 (segment (start 124.354 116.96353) (end 125 116.31753) (width 0.2) (layer "F.Cu") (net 4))
 (segment (start 96.68025 75.95575) (end 101.97275 75.95575) (width 0.2) (layer "F.Cu") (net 4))
 (segment (start 128.0885 73.343374) (end 119.804126 65.059) (width 0.2) (layer "F.Cu") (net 4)))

